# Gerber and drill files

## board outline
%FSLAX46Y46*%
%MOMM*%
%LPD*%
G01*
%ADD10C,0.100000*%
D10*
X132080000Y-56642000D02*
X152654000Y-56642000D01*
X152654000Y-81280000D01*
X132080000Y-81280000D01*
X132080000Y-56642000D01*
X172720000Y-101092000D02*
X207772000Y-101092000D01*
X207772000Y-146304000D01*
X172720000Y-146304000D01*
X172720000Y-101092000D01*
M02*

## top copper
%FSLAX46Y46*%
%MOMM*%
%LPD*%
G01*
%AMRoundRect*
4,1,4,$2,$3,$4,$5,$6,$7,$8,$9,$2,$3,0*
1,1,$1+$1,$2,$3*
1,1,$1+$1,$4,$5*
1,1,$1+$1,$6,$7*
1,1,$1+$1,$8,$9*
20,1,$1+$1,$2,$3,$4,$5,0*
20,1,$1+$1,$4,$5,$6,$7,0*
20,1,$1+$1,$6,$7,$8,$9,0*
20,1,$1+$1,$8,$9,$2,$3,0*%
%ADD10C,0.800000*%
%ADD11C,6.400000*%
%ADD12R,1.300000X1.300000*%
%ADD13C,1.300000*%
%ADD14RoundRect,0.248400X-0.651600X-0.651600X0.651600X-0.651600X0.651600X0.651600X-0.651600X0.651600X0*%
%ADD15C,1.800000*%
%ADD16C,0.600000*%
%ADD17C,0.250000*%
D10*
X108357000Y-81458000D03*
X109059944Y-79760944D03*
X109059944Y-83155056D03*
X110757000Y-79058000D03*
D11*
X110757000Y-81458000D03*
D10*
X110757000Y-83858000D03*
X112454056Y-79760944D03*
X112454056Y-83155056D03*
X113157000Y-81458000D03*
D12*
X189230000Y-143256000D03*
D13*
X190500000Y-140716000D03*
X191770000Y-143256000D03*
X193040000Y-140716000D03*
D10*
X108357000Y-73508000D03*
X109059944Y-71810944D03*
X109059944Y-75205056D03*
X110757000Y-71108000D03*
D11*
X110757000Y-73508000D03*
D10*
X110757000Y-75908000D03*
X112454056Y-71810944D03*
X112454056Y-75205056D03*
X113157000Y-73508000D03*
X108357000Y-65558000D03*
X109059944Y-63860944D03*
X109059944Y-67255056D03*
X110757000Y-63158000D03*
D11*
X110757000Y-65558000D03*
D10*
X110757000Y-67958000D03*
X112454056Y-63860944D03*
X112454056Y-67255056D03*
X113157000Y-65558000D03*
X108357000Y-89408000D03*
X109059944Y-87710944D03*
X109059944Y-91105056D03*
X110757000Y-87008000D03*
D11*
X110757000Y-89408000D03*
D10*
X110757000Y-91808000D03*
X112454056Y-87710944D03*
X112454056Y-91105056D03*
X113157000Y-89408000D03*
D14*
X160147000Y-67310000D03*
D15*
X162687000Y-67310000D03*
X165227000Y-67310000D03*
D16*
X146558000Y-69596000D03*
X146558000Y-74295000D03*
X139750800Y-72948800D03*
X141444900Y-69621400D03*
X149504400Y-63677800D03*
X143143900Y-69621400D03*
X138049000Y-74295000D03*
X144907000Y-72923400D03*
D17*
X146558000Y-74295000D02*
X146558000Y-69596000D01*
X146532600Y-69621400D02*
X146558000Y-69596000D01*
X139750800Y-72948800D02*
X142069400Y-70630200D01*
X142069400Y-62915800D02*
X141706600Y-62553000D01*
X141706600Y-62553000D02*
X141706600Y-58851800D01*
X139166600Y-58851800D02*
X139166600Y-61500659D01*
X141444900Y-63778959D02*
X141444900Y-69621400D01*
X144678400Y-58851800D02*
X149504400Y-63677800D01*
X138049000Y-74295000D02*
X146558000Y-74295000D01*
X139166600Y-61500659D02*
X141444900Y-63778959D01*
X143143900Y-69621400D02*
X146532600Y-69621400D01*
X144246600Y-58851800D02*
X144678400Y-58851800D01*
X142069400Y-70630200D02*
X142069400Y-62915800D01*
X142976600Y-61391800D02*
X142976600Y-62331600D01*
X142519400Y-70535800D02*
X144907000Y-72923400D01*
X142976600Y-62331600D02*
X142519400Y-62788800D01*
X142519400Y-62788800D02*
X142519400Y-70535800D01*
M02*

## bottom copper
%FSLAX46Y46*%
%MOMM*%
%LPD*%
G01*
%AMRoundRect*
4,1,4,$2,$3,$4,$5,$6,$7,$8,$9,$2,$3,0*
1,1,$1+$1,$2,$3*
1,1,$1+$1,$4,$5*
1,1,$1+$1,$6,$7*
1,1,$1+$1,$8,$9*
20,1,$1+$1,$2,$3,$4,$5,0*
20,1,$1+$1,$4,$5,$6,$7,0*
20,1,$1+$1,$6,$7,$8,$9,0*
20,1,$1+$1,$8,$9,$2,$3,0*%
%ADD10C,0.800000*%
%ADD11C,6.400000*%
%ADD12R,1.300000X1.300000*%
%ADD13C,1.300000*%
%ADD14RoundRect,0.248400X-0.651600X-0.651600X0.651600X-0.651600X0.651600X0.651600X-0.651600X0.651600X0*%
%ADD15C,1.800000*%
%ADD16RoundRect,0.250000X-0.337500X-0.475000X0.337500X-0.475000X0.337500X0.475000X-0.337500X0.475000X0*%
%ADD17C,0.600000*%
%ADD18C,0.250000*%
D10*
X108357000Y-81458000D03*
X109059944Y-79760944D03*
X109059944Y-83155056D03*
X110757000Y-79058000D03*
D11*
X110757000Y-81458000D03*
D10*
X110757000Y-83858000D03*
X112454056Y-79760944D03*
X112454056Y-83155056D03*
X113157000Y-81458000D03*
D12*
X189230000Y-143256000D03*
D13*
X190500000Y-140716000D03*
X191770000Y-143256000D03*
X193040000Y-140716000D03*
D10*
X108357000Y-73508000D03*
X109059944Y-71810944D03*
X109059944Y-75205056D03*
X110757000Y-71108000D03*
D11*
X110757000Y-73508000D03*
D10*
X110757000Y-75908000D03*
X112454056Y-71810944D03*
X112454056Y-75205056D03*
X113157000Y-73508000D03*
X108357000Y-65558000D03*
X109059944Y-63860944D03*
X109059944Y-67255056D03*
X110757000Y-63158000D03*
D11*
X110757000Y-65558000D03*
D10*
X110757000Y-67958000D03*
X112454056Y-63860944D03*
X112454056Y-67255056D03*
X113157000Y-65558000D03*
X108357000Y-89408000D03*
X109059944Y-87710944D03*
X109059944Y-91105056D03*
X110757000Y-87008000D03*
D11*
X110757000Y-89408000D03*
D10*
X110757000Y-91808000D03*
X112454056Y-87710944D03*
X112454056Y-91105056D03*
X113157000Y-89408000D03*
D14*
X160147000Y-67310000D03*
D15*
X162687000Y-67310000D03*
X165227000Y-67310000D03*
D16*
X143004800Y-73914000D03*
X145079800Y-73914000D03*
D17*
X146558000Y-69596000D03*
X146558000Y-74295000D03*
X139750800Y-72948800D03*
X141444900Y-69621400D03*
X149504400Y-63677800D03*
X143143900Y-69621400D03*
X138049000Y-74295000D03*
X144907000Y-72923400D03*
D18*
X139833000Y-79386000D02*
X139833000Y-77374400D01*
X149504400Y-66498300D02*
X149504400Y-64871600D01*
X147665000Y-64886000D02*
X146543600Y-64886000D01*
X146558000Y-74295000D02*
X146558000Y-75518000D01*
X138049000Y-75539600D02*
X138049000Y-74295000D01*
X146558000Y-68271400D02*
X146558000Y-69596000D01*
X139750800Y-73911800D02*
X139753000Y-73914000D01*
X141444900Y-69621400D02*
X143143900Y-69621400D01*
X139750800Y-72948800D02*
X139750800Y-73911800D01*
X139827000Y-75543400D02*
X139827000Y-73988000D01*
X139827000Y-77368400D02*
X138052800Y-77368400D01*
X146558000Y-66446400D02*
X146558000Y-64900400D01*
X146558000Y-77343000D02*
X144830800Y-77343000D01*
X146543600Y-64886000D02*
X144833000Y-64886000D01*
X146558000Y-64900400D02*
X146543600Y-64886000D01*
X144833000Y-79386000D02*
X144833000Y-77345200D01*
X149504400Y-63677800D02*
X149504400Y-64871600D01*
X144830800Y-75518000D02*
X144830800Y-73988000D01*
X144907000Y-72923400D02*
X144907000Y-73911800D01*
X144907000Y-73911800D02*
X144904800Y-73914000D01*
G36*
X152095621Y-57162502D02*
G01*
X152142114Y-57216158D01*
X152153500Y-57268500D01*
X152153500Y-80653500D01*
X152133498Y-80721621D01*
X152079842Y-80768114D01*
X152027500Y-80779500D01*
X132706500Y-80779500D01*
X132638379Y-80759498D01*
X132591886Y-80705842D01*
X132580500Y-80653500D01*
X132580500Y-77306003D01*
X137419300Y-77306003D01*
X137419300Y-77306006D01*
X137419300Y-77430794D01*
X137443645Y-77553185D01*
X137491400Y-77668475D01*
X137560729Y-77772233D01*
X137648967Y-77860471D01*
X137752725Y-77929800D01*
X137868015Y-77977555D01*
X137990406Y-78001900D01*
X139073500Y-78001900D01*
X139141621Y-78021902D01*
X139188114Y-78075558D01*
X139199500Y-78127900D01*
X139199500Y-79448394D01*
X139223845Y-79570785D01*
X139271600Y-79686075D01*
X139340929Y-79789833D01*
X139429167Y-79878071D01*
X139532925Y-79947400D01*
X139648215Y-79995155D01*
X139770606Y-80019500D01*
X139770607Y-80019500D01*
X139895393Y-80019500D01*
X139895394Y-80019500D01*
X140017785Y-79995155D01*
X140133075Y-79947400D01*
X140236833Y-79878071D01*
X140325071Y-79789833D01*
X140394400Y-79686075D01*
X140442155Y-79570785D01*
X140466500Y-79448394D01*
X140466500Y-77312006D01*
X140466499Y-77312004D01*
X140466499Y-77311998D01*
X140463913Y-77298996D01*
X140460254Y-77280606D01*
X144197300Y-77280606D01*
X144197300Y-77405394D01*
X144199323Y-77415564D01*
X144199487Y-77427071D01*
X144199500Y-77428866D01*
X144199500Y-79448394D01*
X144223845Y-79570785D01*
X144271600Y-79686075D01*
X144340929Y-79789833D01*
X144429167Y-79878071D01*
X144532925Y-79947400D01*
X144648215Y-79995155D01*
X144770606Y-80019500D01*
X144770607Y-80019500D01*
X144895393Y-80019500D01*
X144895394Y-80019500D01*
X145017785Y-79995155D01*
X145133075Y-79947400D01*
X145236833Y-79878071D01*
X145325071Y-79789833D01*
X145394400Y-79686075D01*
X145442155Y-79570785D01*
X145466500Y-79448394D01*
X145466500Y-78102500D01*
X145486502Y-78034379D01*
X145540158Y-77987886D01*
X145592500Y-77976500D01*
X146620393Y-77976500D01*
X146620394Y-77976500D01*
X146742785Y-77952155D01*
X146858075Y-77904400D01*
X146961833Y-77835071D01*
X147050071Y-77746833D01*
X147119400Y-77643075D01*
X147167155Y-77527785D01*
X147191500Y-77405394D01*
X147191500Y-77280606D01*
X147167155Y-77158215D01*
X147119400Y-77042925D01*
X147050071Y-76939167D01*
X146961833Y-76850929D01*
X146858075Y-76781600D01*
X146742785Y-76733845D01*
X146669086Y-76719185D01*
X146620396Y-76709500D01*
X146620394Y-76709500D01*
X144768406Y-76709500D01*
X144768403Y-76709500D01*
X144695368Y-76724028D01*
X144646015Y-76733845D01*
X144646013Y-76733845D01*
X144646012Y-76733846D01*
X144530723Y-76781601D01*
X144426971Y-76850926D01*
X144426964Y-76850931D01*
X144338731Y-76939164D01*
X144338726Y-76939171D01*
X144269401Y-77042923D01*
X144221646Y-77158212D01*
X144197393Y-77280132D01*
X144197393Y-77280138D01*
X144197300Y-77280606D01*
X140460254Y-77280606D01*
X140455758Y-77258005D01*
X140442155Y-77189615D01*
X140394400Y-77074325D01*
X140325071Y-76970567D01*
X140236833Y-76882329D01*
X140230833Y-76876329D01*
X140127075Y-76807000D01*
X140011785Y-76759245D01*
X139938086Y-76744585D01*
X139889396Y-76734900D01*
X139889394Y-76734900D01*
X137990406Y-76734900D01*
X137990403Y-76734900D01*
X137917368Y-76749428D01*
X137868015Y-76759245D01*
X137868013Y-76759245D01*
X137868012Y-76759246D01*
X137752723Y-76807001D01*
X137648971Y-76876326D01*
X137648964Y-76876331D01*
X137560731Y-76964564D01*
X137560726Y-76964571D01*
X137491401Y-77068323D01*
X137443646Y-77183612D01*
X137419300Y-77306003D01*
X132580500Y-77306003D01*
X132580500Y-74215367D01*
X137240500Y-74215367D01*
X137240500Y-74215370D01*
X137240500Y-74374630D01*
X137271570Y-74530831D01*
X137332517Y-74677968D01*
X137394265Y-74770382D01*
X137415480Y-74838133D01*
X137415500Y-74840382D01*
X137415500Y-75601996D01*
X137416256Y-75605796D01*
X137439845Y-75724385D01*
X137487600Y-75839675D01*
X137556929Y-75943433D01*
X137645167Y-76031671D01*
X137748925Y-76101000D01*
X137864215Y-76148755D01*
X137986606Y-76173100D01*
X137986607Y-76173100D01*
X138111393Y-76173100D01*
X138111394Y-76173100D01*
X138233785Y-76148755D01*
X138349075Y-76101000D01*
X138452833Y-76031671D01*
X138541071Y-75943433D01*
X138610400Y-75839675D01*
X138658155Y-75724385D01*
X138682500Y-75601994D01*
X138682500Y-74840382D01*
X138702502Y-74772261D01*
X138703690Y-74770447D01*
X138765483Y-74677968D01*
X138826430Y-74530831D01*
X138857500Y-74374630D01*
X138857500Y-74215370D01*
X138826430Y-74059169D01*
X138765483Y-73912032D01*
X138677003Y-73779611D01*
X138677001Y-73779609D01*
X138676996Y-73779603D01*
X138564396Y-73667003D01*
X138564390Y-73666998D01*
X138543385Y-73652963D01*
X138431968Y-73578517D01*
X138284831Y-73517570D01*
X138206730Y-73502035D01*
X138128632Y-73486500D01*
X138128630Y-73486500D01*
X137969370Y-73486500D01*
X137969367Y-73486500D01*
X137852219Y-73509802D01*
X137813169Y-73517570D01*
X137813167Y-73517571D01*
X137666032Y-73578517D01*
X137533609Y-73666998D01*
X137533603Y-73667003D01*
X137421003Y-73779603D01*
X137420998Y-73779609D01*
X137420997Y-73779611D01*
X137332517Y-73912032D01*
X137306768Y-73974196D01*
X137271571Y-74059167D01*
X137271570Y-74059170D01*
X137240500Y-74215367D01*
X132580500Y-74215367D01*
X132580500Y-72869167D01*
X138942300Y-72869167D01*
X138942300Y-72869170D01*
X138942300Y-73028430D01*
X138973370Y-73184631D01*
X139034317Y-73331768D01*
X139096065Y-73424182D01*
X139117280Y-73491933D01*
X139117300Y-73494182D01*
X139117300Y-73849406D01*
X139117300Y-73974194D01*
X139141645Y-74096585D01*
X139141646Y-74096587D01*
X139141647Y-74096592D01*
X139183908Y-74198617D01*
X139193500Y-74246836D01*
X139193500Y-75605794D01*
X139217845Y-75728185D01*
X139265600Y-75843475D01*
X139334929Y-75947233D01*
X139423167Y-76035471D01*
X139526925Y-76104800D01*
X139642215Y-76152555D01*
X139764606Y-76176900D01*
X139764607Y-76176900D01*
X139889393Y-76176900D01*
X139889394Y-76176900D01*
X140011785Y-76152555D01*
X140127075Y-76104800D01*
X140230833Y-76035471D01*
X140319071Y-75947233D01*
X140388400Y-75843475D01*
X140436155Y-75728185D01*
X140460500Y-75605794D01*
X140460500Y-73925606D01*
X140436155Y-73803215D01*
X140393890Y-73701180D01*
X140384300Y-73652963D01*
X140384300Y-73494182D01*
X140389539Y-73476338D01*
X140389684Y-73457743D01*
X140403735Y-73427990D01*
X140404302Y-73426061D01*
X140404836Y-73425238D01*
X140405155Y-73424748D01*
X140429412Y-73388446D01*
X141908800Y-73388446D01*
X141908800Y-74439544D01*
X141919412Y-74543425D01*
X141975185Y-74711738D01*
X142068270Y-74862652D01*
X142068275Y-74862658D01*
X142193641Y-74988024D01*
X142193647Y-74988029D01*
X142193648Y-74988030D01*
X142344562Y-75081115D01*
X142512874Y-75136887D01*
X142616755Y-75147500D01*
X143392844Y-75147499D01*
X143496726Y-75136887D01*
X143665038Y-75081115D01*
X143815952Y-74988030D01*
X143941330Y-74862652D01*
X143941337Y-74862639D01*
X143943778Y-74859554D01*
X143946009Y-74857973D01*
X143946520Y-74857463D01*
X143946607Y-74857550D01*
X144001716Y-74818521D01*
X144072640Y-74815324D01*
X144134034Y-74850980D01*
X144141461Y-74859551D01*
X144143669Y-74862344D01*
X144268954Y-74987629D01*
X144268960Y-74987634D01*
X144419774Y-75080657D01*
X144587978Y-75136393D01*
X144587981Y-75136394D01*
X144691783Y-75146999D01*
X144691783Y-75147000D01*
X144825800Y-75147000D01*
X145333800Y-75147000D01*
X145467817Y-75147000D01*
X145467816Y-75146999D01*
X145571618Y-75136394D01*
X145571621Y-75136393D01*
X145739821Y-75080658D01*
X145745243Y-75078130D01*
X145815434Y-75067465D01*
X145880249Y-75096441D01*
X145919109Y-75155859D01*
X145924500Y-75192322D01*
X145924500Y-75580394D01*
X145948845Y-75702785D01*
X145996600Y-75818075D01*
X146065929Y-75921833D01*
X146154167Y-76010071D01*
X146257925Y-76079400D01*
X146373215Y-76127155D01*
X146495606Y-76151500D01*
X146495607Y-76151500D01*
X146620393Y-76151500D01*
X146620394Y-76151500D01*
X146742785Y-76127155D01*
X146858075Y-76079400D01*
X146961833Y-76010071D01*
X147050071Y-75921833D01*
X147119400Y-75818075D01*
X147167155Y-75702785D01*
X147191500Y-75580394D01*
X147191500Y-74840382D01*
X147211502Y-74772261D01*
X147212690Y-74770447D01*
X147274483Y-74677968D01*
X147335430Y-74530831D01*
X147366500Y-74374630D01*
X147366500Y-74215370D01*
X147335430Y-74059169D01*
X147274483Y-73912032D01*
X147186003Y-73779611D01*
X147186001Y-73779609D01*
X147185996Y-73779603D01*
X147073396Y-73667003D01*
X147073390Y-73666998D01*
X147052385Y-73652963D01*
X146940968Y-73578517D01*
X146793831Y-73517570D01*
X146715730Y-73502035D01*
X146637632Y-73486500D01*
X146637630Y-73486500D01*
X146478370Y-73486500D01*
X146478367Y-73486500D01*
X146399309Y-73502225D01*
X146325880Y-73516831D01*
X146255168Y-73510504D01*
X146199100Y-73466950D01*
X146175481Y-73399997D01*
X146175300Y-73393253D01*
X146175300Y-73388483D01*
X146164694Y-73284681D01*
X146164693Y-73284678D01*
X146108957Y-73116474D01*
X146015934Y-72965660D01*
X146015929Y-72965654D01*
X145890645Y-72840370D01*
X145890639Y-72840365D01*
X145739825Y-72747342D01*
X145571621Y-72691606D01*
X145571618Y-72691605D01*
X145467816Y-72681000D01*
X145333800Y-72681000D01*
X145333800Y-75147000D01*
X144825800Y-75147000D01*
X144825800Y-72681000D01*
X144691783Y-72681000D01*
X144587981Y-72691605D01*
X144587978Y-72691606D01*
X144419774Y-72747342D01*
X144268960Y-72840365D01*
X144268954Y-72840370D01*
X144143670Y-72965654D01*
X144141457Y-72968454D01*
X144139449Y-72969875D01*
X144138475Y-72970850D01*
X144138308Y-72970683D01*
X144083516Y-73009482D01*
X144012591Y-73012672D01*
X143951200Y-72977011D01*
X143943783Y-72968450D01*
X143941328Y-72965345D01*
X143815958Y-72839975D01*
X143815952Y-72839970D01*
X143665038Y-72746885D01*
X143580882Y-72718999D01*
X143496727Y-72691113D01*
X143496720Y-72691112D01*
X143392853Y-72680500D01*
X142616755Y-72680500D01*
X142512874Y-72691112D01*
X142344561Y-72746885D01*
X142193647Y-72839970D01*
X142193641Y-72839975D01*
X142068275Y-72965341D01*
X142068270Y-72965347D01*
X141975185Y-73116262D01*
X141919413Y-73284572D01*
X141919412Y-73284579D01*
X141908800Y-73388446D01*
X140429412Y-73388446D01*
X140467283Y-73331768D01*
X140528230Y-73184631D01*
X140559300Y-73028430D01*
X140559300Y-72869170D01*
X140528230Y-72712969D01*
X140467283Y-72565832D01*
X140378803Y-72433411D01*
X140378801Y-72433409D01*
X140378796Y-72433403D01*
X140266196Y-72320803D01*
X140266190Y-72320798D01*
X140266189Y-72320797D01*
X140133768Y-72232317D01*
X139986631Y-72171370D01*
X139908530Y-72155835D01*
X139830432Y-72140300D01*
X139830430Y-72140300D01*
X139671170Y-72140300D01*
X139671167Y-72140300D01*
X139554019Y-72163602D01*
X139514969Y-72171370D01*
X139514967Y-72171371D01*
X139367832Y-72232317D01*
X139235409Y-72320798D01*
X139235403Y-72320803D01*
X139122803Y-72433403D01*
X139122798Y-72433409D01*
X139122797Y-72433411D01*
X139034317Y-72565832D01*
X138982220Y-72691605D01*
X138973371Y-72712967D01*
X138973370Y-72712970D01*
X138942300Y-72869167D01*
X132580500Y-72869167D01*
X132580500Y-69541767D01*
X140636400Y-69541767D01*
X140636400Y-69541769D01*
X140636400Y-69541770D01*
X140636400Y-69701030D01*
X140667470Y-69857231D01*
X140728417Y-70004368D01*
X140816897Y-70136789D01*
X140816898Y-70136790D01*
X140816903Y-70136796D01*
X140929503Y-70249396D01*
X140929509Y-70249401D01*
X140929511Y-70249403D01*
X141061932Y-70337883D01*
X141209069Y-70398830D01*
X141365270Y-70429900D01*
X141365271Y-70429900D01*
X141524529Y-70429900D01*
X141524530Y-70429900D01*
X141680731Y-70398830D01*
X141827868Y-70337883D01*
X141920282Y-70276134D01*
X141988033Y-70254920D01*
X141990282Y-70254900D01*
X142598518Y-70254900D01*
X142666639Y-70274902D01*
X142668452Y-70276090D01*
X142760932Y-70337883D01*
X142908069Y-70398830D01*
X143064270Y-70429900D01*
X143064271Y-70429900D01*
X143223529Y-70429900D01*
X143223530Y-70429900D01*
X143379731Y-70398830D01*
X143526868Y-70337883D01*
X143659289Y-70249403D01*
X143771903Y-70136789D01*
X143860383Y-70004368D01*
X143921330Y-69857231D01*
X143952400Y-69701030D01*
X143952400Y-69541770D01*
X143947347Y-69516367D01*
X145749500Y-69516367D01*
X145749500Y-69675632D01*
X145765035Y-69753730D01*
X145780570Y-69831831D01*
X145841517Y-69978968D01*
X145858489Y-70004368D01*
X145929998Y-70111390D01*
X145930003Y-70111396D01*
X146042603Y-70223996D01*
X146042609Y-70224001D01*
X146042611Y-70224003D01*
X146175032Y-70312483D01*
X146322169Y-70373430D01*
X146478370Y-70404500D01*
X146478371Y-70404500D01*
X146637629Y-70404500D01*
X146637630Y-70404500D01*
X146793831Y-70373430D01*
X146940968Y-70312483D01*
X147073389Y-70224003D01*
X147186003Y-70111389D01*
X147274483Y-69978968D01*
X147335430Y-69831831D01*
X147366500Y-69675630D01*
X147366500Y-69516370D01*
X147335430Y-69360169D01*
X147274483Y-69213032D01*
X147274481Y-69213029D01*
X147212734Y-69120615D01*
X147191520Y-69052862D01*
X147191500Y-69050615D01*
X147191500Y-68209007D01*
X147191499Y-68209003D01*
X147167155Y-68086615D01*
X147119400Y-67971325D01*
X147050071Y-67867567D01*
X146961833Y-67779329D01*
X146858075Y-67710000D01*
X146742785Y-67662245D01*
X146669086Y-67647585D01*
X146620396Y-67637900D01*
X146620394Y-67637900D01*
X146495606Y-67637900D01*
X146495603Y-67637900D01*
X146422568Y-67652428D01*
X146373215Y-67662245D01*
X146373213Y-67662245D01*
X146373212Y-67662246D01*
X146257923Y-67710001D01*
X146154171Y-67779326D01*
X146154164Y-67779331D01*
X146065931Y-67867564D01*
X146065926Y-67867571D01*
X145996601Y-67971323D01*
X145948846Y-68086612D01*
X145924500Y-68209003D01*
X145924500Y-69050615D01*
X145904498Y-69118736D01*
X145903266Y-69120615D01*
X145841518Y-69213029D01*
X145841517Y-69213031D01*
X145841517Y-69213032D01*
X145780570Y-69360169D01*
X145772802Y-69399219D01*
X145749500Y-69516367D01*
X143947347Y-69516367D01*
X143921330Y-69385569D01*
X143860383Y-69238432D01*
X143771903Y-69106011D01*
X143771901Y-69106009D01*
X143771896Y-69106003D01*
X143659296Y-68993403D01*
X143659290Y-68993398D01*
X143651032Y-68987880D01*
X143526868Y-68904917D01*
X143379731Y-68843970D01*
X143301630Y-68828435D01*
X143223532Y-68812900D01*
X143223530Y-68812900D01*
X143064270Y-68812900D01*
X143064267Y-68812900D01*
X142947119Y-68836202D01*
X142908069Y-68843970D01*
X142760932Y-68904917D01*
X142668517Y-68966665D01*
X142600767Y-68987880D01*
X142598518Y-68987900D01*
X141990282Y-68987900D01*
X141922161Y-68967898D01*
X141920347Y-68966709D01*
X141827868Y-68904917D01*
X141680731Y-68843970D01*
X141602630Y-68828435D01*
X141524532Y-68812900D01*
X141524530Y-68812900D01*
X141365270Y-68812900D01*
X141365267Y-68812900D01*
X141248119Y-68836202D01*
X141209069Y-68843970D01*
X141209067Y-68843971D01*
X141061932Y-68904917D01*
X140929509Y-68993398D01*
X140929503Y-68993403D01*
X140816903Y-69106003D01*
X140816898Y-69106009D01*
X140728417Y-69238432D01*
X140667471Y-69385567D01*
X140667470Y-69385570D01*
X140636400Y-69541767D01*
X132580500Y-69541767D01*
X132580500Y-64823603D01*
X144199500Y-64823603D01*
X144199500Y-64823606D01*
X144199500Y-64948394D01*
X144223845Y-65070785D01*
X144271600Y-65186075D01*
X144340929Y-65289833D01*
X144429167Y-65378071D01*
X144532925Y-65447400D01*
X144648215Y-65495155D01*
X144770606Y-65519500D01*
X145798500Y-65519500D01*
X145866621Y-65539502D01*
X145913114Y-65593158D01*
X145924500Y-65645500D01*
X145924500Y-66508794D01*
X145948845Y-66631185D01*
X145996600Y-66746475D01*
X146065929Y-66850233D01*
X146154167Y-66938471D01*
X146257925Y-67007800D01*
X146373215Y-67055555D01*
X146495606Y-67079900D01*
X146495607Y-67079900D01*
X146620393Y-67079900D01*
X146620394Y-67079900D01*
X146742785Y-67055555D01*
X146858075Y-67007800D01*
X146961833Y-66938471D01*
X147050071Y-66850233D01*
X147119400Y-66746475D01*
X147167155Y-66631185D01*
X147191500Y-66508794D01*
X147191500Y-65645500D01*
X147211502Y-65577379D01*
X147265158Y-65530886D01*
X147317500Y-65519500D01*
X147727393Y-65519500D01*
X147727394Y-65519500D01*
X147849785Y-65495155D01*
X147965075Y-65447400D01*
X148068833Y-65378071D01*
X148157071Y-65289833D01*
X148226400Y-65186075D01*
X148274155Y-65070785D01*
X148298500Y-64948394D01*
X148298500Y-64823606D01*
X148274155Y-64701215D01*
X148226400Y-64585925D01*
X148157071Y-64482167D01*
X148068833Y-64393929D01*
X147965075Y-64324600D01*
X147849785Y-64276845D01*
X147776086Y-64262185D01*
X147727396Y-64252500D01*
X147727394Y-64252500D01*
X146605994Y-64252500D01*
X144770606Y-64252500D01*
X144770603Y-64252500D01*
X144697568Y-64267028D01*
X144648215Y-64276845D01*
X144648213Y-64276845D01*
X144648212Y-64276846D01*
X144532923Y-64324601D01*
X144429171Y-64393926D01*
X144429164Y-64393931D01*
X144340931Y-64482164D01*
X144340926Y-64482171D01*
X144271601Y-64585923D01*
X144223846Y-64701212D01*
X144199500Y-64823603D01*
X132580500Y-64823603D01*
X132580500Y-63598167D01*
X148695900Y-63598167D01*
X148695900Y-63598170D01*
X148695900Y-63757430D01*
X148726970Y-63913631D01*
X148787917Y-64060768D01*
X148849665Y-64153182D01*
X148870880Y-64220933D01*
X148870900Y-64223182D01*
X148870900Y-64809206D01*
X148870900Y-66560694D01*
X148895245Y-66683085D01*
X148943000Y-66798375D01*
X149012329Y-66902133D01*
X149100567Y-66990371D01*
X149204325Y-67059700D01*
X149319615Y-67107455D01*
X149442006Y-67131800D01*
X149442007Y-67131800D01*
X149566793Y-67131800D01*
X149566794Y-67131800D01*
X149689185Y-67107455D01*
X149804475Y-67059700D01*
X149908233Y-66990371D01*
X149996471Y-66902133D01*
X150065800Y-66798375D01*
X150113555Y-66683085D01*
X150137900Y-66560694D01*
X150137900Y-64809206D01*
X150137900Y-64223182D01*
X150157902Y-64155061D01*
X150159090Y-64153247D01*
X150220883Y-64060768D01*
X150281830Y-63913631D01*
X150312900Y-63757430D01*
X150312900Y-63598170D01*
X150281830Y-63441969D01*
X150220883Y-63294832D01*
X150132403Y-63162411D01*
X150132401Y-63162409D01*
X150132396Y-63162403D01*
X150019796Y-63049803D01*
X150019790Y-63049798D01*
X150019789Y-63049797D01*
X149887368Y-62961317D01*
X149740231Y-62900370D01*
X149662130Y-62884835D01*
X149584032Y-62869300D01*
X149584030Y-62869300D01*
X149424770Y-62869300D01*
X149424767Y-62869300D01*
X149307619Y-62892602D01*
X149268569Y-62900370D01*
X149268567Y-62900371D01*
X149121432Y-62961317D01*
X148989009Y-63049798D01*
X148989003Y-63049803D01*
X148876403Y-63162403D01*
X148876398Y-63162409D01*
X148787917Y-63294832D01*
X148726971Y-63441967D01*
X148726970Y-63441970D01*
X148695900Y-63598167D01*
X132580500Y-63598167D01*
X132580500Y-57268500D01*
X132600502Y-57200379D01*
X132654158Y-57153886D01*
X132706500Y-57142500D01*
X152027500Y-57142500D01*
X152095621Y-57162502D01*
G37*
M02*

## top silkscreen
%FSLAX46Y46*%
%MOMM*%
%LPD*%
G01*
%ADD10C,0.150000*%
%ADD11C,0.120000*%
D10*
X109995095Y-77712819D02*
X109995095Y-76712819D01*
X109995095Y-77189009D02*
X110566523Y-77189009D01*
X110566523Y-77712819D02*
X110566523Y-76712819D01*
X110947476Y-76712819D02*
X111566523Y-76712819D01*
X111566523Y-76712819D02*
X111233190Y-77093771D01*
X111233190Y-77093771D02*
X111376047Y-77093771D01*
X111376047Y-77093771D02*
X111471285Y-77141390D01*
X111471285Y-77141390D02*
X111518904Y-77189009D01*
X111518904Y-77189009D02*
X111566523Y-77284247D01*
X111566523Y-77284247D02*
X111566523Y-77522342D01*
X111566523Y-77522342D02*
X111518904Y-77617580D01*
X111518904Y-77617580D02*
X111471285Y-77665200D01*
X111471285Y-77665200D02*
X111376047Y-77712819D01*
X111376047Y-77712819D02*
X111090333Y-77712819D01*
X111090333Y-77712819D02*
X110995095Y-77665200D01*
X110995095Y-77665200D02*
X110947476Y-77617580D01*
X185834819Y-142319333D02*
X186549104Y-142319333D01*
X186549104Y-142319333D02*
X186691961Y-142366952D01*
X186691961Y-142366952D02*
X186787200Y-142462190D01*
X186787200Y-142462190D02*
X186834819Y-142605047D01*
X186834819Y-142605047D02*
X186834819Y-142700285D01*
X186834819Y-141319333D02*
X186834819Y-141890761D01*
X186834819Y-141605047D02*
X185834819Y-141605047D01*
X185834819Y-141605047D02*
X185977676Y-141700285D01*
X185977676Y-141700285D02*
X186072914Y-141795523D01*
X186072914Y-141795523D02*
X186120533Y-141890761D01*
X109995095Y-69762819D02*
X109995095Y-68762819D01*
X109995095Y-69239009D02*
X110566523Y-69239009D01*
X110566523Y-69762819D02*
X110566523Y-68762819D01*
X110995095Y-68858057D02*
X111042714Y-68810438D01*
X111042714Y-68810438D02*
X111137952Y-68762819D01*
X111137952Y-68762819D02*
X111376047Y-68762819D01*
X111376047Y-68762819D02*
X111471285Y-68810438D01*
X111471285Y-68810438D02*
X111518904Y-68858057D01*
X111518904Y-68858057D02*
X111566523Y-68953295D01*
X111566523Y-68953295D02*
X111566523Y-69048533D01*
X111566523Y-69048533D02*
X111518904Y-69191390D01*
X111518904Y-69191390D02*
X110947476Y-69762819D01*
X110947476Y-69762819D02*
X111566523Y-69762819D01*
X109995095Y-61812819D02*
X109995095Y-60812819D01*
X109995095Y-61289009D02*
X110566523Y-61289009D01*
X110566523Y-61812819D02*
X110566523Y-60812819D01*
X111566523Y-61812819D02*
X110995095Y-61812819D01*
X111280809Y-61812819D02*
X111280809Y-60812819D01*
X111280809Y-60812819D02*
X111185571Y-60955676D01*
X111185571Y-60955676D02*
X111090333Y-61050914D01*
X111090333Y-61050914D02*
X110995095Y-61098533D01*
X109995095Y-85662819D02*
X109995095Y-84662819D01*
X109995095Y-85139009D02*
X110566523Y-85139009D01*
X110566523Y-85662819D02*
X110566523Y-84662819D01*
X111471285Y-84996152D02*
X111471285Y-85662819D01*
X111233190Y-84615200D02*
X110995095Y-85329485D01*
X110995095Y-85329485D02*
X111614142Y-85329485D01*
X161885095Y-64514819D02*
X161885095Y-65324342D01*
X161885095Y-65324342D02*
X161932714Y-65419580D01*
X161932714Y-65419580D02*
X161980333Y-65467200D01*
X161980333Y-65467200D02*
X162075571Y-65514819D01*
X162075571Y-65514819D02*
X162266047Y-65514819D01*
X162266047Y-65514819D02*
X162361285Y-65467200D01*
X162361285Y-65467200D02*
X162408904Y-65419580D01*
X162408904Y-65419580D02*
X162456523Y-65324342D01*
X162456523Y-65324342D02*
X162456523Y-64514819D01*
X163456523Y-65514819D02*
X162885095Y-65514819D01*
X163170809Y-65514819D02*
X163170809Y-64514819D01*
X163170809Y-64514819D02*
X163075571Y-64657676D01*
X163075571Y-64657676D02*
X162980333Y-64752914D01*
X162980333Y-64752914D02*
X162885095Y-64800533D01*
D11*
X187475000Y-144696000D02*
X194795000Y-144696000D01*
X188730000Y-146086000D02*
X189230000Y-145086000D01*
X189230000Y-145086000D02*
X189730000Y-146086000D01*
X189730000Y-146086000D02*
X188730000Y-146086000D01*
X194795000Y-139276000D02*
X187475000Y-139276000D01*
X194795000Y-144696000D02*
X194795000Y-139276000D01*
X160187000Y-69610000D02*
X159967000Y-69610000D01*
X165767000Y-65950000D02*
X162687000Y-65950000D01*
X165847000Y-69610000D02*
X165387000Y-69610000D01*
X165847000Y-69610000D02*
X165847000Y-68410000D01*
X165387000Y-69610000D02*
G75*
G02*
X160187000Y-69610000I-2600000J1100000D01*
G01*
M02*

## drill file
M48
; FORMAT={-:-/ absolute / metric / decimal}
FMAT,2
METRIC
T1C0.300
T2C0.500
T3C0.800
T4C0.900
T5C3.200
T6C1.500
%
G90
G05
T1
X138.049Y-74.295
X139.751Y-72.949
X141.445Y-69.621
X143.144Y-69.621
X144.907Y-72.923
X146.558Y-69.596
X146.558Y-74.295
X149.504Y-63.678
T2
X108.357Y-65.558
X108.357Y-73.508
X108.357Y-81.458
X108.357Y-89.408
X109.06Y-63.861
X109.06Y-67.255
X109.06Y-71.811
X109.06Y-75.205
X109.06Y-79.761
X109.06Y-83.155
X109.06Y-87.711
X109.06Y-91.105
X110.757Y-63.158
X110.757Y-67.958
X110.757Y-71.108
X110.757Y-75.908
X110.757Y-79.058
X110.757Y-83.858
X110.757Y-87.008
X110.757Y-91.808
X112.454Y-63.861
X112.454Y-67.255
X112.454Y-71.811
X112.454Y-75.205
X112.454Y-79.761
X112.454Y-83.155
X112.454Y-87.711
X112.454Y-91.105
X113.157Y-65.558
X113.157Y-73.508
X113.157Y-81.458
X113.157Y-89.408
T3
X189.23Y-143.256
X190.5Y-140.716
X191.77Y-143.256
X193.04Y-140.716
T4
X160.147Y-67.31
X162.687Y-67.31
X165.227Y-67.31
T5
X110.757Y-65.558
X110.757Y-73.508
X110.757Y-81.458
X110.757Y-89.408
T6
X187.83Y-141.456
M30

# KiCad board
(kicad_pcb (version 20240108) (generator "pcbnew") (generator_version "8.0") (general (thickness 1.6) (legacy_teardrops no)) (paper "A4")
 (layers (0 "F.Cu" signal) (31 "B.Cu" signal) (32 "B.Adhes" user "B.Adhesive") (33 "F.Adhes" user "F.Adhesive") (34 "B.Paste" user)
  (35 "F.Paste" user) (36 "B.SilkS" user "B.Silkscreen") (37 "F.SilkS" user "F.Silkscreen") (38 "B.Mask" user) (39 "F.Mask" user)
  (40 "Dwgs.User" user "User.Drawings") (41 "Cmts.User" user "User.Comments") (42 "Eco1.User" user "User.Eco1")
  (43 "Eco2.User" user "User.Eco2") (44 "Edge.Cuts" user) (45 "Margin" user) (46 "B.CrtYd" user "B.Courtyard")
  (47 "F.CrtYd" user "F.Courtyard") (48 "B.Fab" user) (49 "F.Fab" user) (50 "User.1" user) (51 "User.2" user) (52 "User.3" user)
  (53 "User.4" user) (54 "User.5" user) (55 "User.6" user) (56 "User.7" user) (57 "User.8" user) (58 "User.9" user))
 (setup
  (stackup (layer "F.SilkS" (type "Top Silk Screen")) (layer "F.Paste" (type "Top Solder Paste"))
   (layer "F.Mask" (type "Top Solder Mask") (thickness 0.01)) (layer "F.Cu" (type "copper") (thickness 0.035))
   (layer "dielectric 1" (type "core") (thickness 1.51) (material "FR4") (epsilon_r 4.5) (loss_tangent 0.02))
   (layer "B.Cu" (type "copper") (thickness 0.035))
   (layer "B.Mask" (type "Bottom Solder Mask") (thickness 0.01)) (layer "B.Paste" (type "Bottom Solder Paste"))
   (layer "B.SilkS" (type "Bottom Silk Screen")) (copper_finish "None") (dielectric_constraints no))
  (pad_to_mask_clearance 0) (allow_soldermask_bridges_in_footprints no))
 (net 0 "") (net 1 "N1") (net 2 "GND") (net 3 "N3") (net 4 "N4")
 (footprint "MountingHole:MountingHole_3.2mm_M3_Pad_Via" (layer "F.Cu") (at 110.757 81.458)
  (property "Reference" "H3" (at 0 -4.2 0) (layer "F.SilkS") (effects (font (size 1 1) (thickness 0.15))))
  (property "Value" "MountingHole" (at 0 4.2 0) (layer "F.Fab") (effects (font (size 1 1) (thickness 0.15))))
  (pad "1" thru_hole circle (at -2.4 0) (size 0.8 0.8) (drill 0.5) (layers "*.Cu" "*.Mask") (remove_unused_layers no) (zone_connect 2))
  (pad "1" thru_hole circle (at -1.697056 -1.697056) (size 0.8 0.8) (drill 0.5) (layers "*.Cu" "*.Mask") (remove_unused_layers no)
   (zone_connect 2))
  (pad "1" thru_hole circle (at -1.697056 1.697056) (size 0.8 0.8) (drill 0.5) (layers "*.Cu" "*.Mask") (remove_unused_layers no)
   (zone_connect 2))
  (pad "1" thru_hole circle (at 0 -2.4) (size 0.8 0.8) (drill 0.5) (layers "*.Cu" "*.Mask") (remove_unused_layers no) (zone_connect 2))
  (pad "1" thru_hole circle (at 0 0) (size 6.4 6.4) (drill 3.2) (layers "*.Cu" "*.Mask") (remove_unused_layers no))
  (pad "1" thru_hole circle (at 0 2.4) (size 0.8 0.8) (drill 0.5) (layers "*.Cu" "*.Mask") (remove_unused_layers no) (zone_connect 2))
  (pad "1" thru_hole circle (at 1.697056 -1.697056) (size 0.8 0.8) (drill 0.5) (layers "*.Cu" "*.Mask") (remove_unused_layers no)
   (zone_connect 2))
  (pad "1" thru_hole circle (at 1.697056 1.697056) (size 0.8 0.8) (drill 0.5) (layers "*.Cu" "*.Mask") (remove_unused_layers no)
   (zone_connect 2))
  (pad "1" thru_hole circle (at 2.4 0) (size 0.8 0.8) (drill 0.5) (layers "*.Cu" "*.Mask") (remove_unused_layers no) (zone_connect 2)))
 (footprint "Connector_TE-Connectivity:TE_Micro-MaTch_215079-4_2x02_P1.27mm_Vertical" (layer "F.Cu") (at 189.23 143.256 90)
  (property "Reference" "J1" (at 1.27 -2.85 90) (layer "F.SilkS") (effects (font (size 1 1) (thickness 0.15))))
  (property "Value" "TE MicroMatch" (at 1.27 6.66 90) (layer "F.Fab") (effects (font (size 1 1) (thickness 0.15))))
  (fp_line (start -1.44 -1.755) (end -1.44 5.565) (stroke (width 0.12) (type solid)) (layer "F.SilkS"))
  (fp_line (start -2.83 -0.5) (end -1.83 0) (stroke (width 0.12) (type solid)) (layer "F.SilkS"))
  (fp_line (start -1.83 0) (end -2.83 0.5) (stroke (width 0.12) (type solid)) (layer "F.SilkS"))
  (fp_line (start -2.83 0.5) (end -2.83 -0.5) (stroke (width 0.12) (type solid)) (layer "F.SilkS"))
  (fp_line (start 3.98 5.565) (end 3.98 -1.755) (stroke (width 0.12) (type solid)) (layer "F.SilkS"))
  (fp_line (start -1.44 5.565) (end 3.98 5.565) (stroke (width 0.12) (type solid)) (layer "F.SilkS"))
  (pad "" np_thru_hole circle (at 1.8 -1.4 90) (size 1.5 1.5) (drill 1.5) (layers "*.Cu" "*.Mask"))
  (pad "1" thru_hole rect (at 0 0 90) (size 1.3 1.3) (drill 0.8) (layers "*.Cu" "*.Mask") (remove_unused_layers no) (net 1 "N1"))
  (pad "2" thru_hole circle (at 2.54 1.27 90) (size 1.3 1.3) (drill 0.8) (layers "*.Cu" "*.Mask") (remove_unused_layers no) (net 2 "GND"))
  (pad "3" thru_hole circle (at 0 2.54 90) (size 1.3 1.3) (drill 0.8) (layers "*.Cu" "*.Mask") (remove_unused_layers no) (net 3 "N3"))
  (pad "4" thru_hole circle (at 2.54 3.81 90) (size 1.3 1.3) (drill 0.8) (layers "*.Cu" "*.Mask") (remove_unused_layers no) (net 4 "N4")))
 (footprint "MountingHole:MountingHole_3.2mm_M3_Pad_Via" (layer "F.Cu") (at 110.757 73.508)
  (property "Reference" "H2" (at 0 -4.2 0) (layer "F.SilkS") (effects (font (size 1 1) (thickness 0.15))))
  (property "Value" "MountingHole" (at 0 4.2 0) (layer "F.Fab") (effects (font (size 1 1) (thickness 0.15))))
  (pad "1" thru_hole circle (at -2.4 0) (size 0.8 0.8) (drill 0.5) (layers "*.Cu" "*.Mask") (remove_unused_layers no) (zone_connect 2))
  (pad "1" thru_hole circle (at -1.697056 -1.697056) (size 0.8 0.8) (drill 0.5) (layers "*.Cu" "*.Mask") (remove_unused_layers no)
   (zone_connect 2))
  (pad "1" thru_hole circle (at -1.697056 1.697056) (size 0.8 0.8) (drill 0.5) (layers "*.Cu" "*.Mask") (remove_unused_layers no)
   (zone_connect 2))
  (pad "1" thru_hole circle (at 0 -2.4) (size 0.8 0.8) (drill 0.5) (layers "*.Cu" "*.Mask") (remove_unused_layers no) (zone_connect 2))
  (pad "1" thru_hole circle (at 0 0) (size 6.4 6.4) (drill 3.2) (layers "*.Cu" "*.Mask") (remove_unused_layers no))
  (pad "1" thru_hole circle (at 0 2.4) (size 0.8 0.8) (drill 0.5) (layers "*.Cu" "*.Mask") (remove_unused_layers no) (zone_connect 2))
  (pad "1" thru_hole circle (at 1.697056 -1.697056) (size 0.8 0.8) (drill 0.5) (layers "*.Cu" "*.Mask") (remove_unused_layers no)
   (zone_connect 2))
  (pad "1" thru_hole circle (at 1.697056 1.697056) (size 0.8 0.8) (drill 0.5) (layers "*.Cu" "*.Mask") (remove_unused_layers no)
   (zone_connect 2))
  (pad "1" thru_hole circle (at 2.4 0) (size 0.8 0.8) (drill 0.5) (layers "*.Cu" "*.Mask") (remove_unused_layers no) (zone_connect 2)))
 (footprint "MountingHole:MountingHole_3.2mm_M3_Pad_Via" (layer "F.Cu") (at 110.757 65.558)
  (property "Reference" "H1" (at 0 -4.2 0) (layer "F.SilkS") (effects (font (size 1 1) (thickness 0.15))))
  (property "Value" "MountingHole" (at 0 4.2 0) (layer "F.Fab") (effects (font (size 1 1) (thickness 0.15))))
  (pad "1" thru_hole circle (at -2.4 0) (size 0.8 0.8) (drill 0.5) (layers "*.Cu" "*.Mask") (remove_unused_layers no) (zone_connect 2))
  (pad "1" thru_hole circle (at -1.697056 -1.697056) (size 0.8 0.8) (drill 0.5) (layers "*.Cu" "*.Mask") (remove_unused_layers no)
   (zone_connect 2))
  (pad "1" thru_hole circle (at -1.697056 1.697056) (size 0.8 0.8) (drill 0.5) (layers "*.Cu" "*.Mask") (remove_unused_layers no)
   (zone_connect 2))
  (pad "1" thru_hole circle (at 0 -2.4) (size 0.8 0.8) (drill 0.5) (layers "*.Cu" "*.Mask") (remove_unused_layers no) (zone_connect 2))
  (pad "1" thru_hole circle (at 0 0) (size 6.4 6.4) (drill 3.2) (layers "*.Cu" "*.Mask") (remove_unused_layers no))
  (pad "1" thru_hole circle (at 0 2.4) (size 0.8 0.8) (drill 0.5) (layers "*.Cu" "*.Mask") (remove_unused_layers no) (zone_connect 2))
  (pad "1" thru_hole circle (at 1.697056 -1.697056) (size 0.8 0.8) (drill 0.5) (layers "*.Cu" "*.Mask") (remove_unused_layers no)
   (zone_connect 2))
  (pad "1" thru_hole circle (at 1.697056 1.697056) (size 0.8 0.8) (drill 0.5) (layers "*.Cu" "*.Mask") (remove_unused_layers no)
   (zone_connect 2))
  (pad "1" thru_hole circle (at 2.4 0) (size 0.8 0.8) (drill 0.5) (layers "*.Cu" "*.Mask") (remove_unused_layers no) (zone_connect 2)))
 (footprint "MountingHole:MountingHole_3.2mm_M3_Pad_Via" (layer "F.Cu") (at 110.757 89.408)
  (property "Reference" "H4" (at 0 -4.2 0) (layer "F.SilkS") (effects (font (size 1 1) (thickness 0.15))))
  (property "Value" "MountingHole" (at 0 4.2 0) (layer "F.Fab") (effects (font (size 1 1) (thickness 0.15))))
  (pad "1" thru_hole circle (at -2.4 0) (size 0.8 0.8) (drill 0.5) (layers "*.Cu" "*.Mask") (remove_unused_layers no) (zone_connect 2))
  (pad "1" thru_hole circle (at -1.697056 -1.697056) (size 0.8 0.8) (drill 0.5) (layers "*.Cu" "*.Mask") (remove_unused_layers no)
   (zone_connect 2))
  (pad "1" thru_hole circle (at -1.697056 1.697056) (size 0.8 0.8) (drill 0.5) (layers "*.Cu" "*.Mask") (remove_unused_layers no)
   (zone_connect 2))
  (pad "1" thru_hole circle (at 0 -2.4) (size 0.8 0.8) (drill 0.5) (layers "*.Cu" "*.Mask") (remove_unused_layers no) (zone_connect 2))
  (pad "1" thru_hole circle (at 0 0) (size 6.4 6.4) (drill 3.2) (layers "*.Cu" "*.Mask") (remove_unused_layers no))
  (pad "1" thru_hole circle (at 0 2.4) (size 0.8 0.8) (drill 0.5) (layers "*.Cu" "*.Mask") (remove_unused_layers no) (zone_connect 2))
  (pad "1" thru_hole circle (at 1.697056 -1.697056) (size 0.8 0.8) (drill 0.5) (layers "*.Cu" "*.Mask") (remove_unused_layers no)
   (zone_connect 2))
  (pad "1" thru_hole circle (at 1.697056 1.697056) (size 0.8 0.8) (drill 0.5) (layers "*.Cu" "*.Mask") (remove_unused_layers no)
   (zone_connect 2))
  (pad "1" thru_hole circle (at 2.4 0) (size 0.8 0.8) (drill 0.5) (layers "*.Cu" "*.Mask") (remove_unused_layers no) (zone_connect 2)))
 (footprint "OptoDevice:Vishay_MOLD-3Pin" (layer "F.Cu") (at 160.147 67.31)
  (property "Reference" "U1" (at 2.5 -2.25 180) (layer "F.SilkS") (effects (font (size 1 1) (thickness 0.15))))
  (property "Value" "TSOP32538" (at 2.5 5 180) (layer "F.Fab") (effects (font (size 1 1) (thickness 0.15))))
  (fp_line (start 0.04 2.3) (end -0.18 2.3) (stroke (width 0.12) (type solid)) (layer "F.SilkS"))
  (fp_line (start 5.62 -1.36) (end 2.54 -1.36) (stroke (width 0.12) (type solid)) (layer "F.SilkS"))
  (fp_line (start 5.7 2.3) (end 5.24 2.3) (stroke (width 0.12) (type solid)) (layer "F.SilkS"))
  (fp_line (start 5.7 2.3) (end 5.7 1.1) (stroke (width 0.12) (type solid)) (layer "F.SilkS"))
  (fp_arc (start 5.24 2.3) (mid 2.64 4.023119) (end 0.04 2.3) (stroke (width 0.12) (type solid)) (layer "F.SilkS"))
  (pad "1" thru_hole roundrect (at 0 0) (size 1.8 1.8) (drill 0.9) (layers "*.Cu" "*.Mask") (remove_unused_layers no)
   (roundrect_rratio 0.138) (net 3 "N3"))
  (pad "2" thru_hole circle (at 2.54 0) (size 1.8 1.8) (drill 0.9) (layers "*.Cu" "*.Mask") (remove_unused_layers no) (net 1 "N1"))
  (pad "3" thru_hole circle (at 5.08 0) (size 1.8 1.8) (drill 0.9) (layers "*.Cu" "*.Mask") (remove_unused_layers no) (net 2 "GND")))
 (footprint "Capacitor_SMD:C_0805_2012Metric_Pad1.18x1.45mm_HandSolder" (layer "B.Cu") (at 144.0423 73.914)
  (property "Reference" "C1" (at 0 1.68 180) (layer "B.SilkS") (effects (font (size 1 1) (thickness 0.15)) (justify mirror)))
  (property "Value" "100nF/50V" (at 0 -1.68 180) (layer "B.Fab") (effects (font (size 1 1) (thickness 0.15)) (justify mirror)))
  (pad "1" smd roundrect (at -1.0375 0) (size 1.175 1.45) (layers "B.Cu" "B.Paste" "B.Mask") (roundrect_rratio 0.212766) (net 1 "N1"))
  (pad "2" smd roundrect (at 1.0375 0) (size 1.175 1.45) (layers "B.Cu" "B.Paste" "B.Mask") (roundrect_rratio 0.212766) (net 2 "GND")))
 (gr_rect (start 132.08 56.642) (end 152.654 81.28) (stroke (width 0.1) (type solid)) (fill none) (layer "Edge.Cuts"))
 (gr_rect (start 172.72 101.092) (end 207.772 146.304) (stroke (width 0.1) (type default)) (fill none) (layer "Edge.Cuts"))
 (segment (start 146.558 74.295) (end 146.558 69.596) (width 0.25) (layer "F.Cu") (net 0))
 (segment (start 146.5326 69.6214) (end 146.558 69.596) (width 0.25) (layer "F.Cu") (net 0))
 (segment (start 139.7508 72.9488) (end 142.0694 70.6302) (width 0.25) (layer "F.Cu") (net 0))
 (segment (start 142.0694 62.9158) (end 141.7066 62.553) (width 0.25) (layer "F.Cu") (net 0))
 (segment (start 141.7066 62.553) (end 141.7066 58.8518) (width 0.25) (layer "F.Cu") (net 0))
 (segment (start 139.1666 58.8518) (end 139.1666 61.500659) (width 0.25) (layer "F.Cu") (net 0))
 (segment (start 141.4449 63.778959) (end 141.4449 69.6214) (width 0.25) (layer "F.Cu") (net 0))
 (segment (start 144.6784 58.8518) (end 149.5044 63.6778) (width 0.25) (layer "F.Cu") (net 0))
 (segment (start 138.049 74.295) (end 146.558 74.295) (width 0.25) (layer "F.Cu") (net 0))
 (segment (start 139.1666 61.500659) (end 141.4449 63.778959) (width 0.25) (layer "F.Cu") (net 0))
 (segment (start 143.1439 69.6214) (end 146.5326 69.6214) (width 0.25) (layer "F.Cu") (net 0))
 (segment (start 144.2466 58.8518) (end 144.6784 58.8518) (width 0.25) (layer "F.Cu") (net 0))
 (segment (start 142.0694 70.6302) (end 142.0694 62.9158) (width 0.25) (layer "F.Cu") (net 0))
 (via (at 146.558 69.596) (size 0.6) (drill 0.3) (layers "F.Cu" "B.Cu") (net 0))
 (via (at 146.558 74.295) (size 0.6) (drill 0.3) (layers "F.Cu" "B.Cu") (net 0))
 (via (at 139.7508 72.9488) (size 0.6) (drill 0.3) (layers "F.Cu" "B.Cu") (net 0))
 (via (at 141.4449 69.6214) (size 0.6) (drill 0.3) (layers "F.Cu" "B.Cu") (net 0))
 (via (at 149.5044 63.6778) (size 0.6) (drill 0.3) (layers "F.Cu" "B.Cu") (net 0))
 (via (at 143.1439 69.6214) (size 0.6) (drill 0.3) (layers "F.Cu" "B.Cu") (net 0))
 (via (at 138.049 74.295) (size 0.6) (drill 0.3) (layers "F.Cu" "B.Cu") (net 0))
 (segment (start 139.833 79.386) (end 139.833 77.3744) (width 0.25) (layer "B.Cu") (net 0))
 (segment (start 149.5044 66.4983) (end 149.5044 64.8716) (width 0.25) (layer "B.Cu") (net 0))
 (segment (start 147.665 64.886) (end 146.5436 64.886) (width 0.25) (layer "B.Cu") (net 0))
 (segment (start 146.558 74.295) (end 146.558 75.518) (width 0.25) (layer "B.Cu") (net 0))
 (segment (start 138.049 75.5396) (end 138.049 74.295) (width 0.25) (layer "B.Cu") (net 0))
 (segment (start 146.558 68.2714) (end 146.558 69.596) (width 0.25) (layer "B.Cu") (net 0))
 (segment (start 139.7508 73.9118) (end 139.753 73.914) (width 0.25) (layer "B.Cu") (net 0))
 (segment (start 141.4449 69.6214) (end 143.1439 69.6214) (width 0.25) (layer "B.Cu") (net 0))
 (segment (start 139.7508 72.9488) (end 139.7508 73.9118) (width 0.25) (layer "B.Cu") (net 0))
 (segment (start 139.827 75.5434) (end 139.827 73.988) (width 0.25) (layer "B.Cu") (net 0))
 (segment (start 139.827 77.3684) (end 138.0528 77.3684) (width 0.25) (layer "B.Cu") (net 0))
 (segment (start 146.558 66.4464) (end 146.558 64.9004) (width 0.25) (layer "B.Cu") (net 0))
 (segment (start 146.558 77.343) (end 144.8308 77.343) (width 0.25) (layer "B.Cu") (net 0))
 (segment (start 146.5436 64.886) (end 144.833 64.886) (width 0.25) (layer "B.Cu") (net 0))
 (segment (start 146.558 64.9004) (end 146.5436 64.886) (width 0.25) (layer "B.Cu") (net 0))
 (segment (start 144.833 79.386) (end 144.833 77.3452) (width 0.25) (layer "B.Cu") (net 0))
 (segment (start 149.5044 63.6778) (end 149.5044 64.8716) (width 0.25) (layer "B.Cu") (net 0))
 (segment (start 142.9766 61.3918) (end 142.9766 62.3316) (width 0.25) (layer "F.Cu") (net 2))
 (segment (start 142.5194 70.5358) (end 144.907 72.9234) (width 0.25) (layer "F.Cu") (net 2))
 (segment (start 142.9766 62.3316) (end 142.5194 62.7888) (width 0.25) (layer "F.Cu") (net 2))
 (segment (start 142.5194 62.7888) (end 142.5194 70.5358) (width 0.25) (layer "F.Cu") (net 2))
 (via (at 144.907 72.9234) (size 0.6) (drill 0.3) (layers "F.Cu" "B.Cu") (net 2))
 (segment (start 144.8308 75.518) (end 144.8308 73.988) (width 0.25) (layer "B.Cu") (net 2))
 (segment (start 144.907 72.9234) (end 144.907 73.9118) (width 0.25) (layer "B.Cu") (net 2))
 (segment (start 144.907 73.9118) (end 144.9048 73.914) (width 0.25) (layer "B.Cu") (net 2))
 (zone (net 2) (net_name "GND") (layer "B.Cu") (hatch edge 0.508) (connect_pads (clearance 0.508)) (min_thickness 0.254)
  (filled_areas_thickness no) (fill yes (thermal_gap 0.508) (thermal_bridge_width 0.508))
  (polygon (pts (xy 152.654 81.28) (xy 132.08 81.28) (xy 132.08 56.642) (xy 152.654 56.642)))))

